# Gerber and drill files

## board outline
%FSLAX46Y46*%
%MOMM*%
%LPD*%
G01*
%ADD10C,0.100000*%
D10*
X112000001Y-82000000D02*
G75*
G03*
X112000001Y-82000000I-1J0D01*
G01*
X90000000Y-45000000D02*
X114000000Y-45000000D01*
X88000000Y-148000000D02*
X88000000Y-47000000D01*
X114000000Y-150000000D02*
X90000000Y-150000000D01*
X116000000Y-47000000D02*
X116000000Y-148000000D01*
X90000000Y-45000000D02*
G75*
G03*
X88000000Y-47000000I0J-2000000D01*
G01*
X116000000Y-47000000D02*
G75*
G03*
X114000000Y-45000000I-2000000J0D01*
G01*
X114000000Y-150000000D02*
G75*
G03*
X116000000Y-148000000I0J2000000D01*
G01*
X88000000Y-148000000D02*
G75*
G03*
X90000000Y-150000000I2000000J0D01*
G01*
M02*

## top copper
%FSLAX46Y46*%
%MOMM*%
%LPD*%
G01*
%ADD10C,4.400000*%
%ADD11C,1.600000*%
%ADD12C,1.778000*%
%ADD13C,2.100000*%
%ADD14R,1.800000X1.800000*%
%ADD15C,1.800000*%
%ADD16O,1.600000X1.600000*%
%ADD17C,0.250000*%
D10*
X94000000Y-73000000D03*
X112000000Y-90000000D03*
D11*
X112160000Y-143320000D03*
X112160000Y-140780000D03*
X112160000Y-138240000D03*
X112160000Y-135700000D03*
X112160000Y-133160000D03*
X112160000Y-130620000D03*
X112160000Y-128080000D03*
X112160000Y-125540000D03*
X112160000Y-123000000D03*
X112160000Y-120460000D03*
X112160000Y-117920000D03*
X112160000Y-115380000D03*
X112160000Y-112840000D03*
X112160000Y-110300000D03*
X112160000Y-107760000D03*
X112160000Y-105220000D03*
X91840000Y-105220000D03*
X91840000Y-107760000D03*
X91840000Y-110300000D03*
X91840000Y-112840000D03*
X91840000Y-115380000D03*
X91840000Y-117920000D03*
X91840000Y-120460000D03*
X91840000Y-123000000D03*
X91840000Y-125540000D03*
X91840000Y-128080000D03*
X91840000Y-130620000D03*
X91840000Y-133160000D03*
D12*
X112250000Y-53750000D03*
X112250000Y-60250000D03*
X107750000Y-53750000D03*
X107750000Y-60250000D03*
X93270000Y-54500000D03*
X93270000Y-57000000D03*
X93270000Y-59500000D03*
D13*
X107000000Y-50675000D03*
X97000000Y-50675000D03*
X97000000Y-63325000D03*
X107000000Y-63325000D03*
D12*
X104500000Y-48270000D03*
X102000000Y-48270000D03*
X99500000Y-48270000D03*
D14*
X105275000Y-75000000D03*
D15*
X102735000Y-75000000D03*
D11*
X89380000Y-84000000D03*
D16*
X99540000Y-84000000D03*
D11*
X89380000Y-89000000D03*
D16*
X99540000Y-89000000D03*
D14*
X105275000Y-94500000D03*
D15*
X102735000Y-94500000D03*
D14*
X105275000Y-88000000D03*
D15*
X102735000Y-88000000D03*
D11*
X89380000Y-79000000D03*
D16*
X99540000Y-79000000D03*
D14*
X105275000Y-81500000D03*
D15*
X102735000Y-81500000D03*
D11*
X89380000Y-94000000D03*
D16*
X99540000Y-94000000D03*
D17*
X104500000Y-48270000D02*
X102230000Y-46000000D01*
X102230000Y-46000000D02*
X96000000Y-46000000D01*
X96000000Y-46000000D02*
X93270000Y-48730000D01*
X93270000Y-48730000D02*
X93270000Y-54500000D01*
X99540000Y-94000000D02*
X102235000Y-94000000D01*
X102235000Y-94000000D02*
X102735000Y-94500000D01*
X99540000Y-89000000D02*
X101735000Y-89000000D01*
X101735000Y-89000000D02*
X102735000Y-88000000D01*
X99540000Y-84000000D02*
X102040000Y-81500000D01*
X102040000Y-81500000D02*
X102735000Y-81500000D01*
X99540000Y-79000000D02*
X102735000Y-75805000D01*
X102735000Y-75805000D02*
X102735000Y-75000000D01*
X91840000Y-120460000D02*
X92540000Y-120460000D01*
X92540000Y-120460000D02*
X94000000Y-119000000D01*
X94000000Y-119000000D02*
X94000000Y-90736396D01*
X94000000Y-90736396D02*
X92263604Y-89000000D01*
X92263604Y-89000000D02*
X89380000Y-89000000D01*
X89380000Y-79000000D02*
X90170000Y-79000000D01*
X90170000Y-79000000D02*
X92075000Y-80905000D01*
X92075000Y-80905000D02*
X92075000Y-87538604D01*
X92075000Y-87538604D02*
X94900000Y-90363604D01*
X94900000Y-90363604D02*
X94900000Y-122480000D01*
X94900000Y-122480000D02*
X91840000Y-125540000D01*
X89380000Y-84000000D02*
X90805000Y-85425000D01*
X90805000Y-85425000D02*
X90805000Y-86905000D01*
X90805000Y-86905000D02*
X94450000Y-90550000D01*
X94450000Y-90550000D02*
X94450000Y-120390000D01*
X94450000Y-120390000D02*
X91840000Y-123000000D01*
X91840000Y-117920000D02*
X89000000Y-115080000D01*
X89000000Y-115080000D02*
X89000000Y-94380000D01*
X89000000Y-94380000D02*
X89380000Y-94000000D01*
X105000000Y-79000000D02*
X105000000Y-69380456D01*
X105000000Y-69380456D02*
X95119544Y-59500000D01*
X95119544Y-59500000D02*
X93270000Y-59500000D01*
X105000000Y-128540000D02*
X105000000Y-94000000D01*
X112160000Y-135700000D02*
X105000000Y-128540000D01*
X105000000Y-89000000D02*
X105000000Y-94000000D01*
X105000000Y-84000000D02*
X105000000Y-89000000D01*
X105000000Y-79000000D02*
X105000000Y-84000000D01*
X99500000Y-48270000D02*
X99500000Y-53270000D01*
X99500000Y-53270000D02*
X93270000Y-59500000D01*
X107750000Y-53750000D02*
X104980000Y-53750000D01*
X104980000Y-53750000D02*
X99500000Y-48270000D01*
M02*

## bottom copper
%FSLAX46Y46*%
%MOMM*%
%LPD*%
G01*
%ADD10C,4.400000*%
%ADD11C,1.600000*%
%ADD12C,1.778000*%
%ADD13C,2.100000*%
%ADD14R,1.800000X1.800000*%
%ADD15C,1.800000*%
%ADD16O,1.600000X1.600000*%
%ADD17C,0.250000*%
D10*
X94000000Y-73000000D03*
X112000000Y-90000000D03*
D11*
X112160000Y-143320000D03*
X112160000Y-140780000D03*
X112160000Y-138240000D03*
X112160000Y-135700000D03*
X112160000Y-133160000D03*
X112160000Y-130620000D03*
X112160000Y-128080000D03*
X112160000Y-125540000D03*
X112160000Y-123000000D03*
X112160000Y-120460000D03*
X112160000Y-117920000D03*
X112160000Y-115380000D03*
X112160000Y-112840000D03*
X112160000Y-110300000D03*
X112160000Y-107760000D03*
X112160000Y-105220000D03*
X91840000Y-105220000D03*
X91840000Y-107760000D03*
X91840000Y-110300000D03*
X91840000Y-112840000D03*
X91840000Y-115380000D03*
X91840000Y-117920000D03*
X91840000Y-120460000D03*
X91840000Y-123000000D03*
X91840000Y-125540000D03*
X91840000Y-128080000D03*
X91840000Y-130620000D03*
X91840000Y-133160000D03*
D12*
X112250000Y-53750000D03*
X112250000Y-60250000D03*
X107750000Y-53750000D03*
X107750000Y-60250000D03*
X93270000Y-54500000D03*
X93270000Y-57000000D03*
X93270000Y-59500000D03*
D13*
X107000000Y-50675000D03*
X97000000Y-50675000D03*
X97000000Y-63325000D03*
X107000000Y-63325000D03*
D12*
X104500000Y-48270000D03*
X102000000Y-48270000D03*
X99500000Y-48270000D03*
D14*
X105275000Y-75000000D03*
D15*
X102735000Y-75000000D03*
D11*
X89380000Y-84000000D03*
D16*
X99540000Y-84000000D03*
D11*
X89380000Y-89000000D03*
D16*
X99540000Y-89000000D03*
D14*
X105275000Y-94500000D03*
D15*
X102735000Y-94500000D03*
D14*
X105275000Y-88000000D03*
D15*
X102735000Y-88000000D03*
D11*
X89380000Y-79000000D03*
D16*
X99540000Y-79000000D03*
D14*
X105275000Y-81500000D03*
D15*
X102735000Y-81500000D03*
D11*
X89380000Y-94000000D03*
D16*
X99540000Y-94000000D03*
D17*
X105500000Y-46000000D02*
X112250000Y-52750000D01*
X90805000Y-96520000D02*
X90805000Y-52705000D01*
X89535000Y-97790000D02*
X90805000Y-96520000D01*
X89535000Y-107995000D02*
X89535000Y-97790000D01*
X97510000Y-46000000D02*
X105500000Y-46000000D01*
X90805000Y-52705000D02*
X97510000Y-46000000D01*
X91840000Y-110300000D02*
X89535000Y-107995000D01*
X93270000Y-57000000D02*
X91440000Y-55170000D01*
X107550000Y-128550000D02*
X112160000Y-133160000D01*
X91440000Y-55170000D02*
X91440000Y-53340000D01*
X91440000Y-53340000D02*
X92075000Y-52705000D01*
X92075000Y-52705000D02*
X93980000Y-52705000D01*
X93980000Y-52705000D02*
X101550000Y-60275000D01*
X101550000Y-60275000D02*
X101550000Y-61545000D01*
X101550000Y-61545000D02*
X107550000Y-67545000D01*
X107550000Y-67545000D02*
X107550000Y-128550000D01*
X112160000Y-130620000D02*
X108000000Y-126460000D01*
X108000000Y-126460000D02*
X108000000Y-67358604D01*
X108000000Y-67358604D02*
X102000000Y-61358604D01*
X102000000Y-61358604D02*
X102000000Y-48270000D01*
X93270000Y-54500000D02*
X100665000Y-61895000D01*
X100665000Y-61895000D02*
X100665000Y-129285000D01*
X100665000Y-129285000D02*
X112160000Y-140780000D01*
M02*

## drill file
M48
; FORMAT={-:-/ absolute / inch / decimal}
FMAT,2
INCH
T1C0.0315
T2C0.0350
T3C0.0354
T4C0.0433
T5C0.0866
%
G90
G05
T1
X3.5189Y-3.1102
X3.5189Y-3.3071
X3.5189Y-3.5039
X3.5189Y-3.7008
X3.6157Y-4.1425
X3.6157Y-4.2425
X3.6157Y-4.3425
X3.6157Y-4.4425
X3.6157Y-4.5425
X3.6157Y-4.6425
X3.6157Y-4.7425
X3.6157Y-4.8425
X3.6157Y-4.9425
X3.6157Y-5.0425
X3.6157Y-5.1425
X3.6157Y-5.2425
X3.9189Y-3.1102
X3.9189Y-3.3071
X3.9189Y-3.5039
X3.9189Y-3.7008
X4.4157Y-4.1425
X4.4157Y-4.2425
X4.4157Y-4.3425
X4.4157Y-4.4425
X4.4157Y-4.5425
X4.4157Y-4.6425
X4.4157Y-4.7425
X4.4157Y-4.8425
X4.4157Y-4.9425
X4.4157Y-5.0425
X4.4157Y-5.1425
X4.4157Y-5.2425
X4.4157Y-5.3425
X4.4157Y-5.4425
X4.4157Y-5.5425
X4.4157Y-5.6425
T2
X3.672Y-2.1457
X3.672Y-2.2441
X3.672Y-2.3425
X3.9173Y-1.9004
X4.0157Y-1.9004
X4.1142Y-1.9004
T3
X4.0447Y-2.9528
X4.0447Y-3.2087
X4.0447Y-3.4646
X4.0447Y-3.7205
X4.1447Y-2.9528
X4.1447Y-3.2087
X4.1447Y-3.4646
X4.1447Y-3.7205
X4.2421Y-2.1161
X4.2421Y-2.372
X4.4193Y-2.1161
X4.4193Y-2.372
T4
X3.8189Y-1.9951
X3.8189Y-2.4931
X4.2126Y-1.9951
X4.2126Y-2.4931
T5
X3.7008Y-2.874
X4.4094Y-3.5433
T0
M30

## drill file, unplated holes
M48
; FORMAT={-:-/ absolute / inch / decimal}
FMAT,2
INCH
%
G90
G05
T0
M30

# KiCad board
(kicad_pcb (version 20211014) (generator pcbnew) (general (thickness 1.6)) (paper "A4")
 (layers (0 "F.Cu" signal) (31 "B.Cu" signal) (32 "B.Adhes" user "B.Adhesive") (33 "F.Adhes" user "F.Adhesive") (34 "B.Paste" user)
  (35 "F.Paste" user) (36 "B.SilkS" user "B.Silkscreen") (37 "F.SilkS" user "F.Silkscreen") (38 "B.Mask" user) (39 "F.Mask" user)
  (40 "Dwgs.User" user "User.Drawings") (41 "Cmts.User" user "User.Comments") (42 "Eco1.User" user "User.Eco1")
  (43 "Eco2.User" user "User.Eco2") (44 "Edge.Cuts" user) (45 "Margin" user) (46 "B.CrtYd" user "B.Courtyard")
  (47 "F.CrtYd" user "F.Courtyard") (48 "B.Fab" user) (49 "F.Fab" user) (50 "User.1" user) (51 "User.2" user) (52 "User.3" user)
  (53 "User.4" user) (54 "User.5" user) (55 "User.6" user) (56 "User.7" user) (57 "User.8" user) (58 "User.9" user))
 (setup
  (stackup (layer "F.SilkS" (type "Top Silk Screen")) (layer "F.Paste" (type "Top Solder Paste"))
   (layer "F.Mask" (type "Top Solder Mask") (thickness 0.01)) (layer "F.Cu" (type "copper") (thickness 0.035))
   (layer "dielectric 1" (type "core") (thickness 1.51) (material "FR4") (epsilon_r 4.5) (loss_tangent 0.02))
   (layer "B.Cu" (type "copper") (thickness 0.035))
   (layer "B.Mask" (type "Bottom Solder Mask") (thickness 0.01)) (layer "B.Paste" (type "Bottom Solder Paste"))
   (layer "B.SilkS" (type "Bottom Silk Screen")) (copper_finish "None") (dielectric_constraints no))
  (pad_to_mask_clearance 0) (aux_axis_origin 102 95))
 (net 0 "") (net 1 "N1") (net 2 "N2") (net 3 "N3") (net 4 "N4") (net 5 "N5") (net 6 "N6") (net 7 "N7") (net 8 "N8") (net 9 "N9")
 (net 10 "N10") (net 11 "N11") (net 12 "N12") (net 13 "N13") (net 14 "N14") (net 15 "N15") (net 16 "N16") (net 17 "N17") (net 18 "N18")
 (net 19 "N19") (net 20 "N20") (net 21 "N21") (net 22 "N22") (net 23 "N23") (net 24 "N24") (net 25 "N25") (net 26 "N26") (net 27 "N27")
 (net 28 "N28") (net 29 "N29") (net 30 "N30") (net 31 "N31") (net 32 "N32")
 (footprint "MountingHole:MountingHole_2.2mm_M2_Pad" (layer "F.Cu") (at 94 73)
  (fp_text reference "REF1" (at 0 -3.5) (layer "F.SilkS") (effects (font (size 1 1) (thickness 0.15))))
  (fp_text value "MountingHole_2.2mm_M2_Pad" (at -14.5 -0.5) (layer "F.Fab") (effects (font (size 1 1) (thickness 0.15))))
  (pad "1" thru_hole circle (at 0 0) (size 4.4 4.4) (drill 2.2) (layers *.Cu *.Mask)))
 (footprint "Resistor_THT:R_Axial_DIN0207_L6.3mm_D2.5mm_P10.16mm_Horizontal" (layer "F.Cu") (at 89.38 84)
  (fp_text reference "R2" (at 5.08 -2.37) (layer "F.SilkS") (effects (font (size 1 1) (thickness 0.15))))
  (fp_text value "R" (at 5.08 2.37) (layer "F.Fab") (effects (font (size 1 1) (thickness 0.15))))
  (pad "1" thru_hole circle (at 0 0) (size 1.6 1.6) (drill 0.8) (layers *.Cu *.Mask) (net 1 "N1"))
  (pad "2" thru_hole oval (at 10.16 0) (size 1.6 1.6) (drill 0.8) (layers *.Cu *.Mask) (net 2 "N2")))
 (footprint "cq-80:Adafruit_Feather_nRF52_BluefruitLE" (layer "F.Cu") (at 102 123 180)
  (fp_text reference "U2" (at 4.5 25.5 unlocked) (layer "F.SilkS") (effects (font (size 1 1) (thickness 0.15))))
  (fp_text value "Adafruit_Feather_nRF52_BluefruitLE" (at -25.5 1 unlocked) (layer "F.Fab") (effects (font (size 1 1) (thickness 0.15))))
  (pad "1" thru_hole circle (at -10.16 -20.32) (size 1.6 1.6) (drill 0.8) (layers *.Cu *.Mask) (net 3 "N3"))
  (pad "2" thru_hole circle (at -10.16 -17.78) (size 1.6 1.6) (drill 0.8) (layers *.Cu *.Mask) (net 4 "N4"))
  (pad "3" thru_hole circle (at -10.16 -15.24) (size 1.6 1.6) (drill 0.8) (layers *.Cu *.Mask) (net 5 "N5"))
  (pad "4" thru_hole circle (at -10.16 -12.7) (size 1.6 1.6) (drill 0.8) (layers *.Cu *.Mask) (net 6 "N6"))
  (pad "5" thru_hole circle (at -10.16 -10.16) (size 1.6 1.6) (drill 0.8) (layers *.Cu *.Mask) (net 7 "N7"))
  (pad "6" thru_hole circle (at -10.16 -7.62) (size 1.6 1.6) (drill 0.8) (layers *.Cu *.Mask) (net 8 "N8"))
  (pad "7" thru_hole circle (at -10.16 -5.08) (size 1.6 1.6) (drill 0.8) (layers *.Cu *.Mask) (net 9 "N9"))
  (pad "8" thru_hole circle (at -10.16 -2.54) (size 1.6 1.6) (drill 0.8) (layers *.Cu *.Mask) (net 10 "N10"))
  (pad "9" thru_hole circle (at -10.16 0) (size 1.6 1.6) (drill 0.8) (layers *.Cu *.Mask) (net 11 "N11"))
  (pad "10" thru_hole circle (at -10.16 2.54) (size 1.6 1.6) (drill 0.8) (layers *.Cu *.Mask) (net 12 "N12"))
  (pad "11" thru_hole circle (at -10.16 5.08) (size 1.6 1.6) (drill 0.8) (layers *.Cu *.Mask) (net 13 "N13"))
  (pad "12" thru_hole circle (at -10.16 7.62) (size 1.6 1.6) (drill 0.8) (layers *.Cu *.Mask) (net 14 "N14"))
  (pad "13" thru_hole circle (at -10.16 10.16) (size 1.6 1.6) (drill 0.8) (layers *.Cu *.Mask) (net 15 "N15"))
  (pad "14" thru_hole circle (at -10.16 12.7) (size 1.6 1.6) (drill 0.8) (layers *.Cu *.Mask) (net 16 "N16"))
  (pad "15" thru_hole circle (at -10.16 15.24) (size 1.6 1.6) (drill 0.8) (layers *.Cu *.Mask) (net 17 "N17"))
  (pad "16" thru_hole circle (at -10.16 17.78) (size 1.6 1.6) (drill 0.8) (layers *.Cu *.Mask) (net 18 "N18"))
  (pad "17" thru_hole circle (at 10.16 17.78) (size 1.6 1.6) (drill 0.8) (layers *.Cu *.Mask) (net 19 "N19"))
  (pad "18" thru_hole circle (at 10.16 15.24) (size 1.6 1.6) (drill 0.8) (layers *.Cu *.Mask) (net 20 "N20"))
  (pad "19" thru_hole circle (at 10.16 12.7) (size 1.6 1.6) (drill 0.8) (layers *.Cu *.Mask) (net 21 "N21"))
  (pad "20" thru_hole circle (at 10.16 10.16) (size 1.6 1.6) (drill 0.8) (layers *.Cu *.Mask) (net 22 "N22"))
  (pad "21" thru_hole circle (at 10.16 7.62) (size 1.6 1.6) (drill 0.8) (layers *.Cu *.Mask) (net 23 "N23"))
  (pad "22" thru_hole circle (at 10.16 5.08) (size 1.6 1.6) (drill 0.8) (layers *.Cu *.Mask) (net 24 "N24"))
  (pad "23" thru_hole circle (at 10.16 2.54) (size 1.6 1.6) (drill 0.8) (layers *.Cu *.Mask) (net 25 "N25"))
  (pad "24" thru_hole circle (at 10.16 0) (size 1.6 1.6) (drill 0.8) (layers *.Cu *.Mask) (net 1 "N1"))
  (pad "25" thru_hole circle (at 10.16 -2.54) (size 1.6 1.6) (drill 0.8) (layers *.Cu *.Mask) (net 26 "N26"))
  (pad "26" thru_hole circle (at 10.16 -5.08) (size 1.6 1.6) (drill 0.8) (layers *.Cu *.Mask) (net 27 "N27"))
  (pad "27" thru_hole circle (at 10.16 -7.62) (size 1.6 1.6) (drill 0.8) (layers *.Cu *.Mask) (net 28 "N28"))
  (pad "28" thru_hole circle (at 10.16 -10.16) (size 1.6 1.6) (drill 0.8) (layers *.Cu *.Mask) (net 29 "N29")))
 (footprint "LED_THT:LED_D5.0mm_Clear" (layer "F.Cu") (at 105.275 75 180)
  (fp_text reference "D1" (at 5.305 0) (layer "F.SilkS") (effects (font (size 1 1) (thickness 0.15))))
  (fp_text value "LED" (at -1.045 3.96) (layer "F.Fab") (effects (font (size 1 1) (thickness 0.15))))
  (pad "1" thru_hole rect (at 0 0 180) (size 1.8 1.8) (drill 0.9) (layers *.Cu *.Mask) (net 6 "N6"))
  (pad "2" thru_hole circle (at 2.54 0 180) (size 1.8 1.8) (drill 0.9) (layers *.Cu *.Mask) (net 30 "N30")))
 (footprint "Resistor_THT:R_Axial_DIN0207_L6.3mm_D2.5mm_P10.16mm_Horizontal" (layer "F.Cu") (at 89.38 89)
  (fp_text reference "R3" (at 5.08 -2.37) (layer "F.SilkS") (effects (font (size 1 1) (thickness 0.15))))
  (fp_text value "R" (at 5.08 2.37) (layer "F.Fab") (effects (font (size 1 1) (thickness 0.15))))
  (pad "1" thru_hole circle (at 0 0) (size 1.6 1.6) (drill 0.8) (layers *.Cu *.Mask) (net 25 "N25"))
  (pad "2" thru_hole oval (at 10.16 0) (size 1.6 1.6) (drill 0.8) (layers *.Cu *.Mask) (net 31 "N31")))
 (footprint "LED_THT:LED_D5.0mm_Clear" (layer "F.Cu") (at 105.275 94.5 180)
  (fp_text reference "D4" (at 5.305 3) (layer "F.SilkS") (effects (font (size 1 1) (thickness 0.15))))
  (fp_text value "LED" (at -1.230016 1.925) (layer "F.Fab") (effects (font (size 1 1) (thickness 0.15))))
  (pad "1" thru_hole rect (at 0 0 180) (size 1.8 1.8) (drill 0.9) (layers *.Cu *.Mask) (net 6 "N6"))
  (pad "2" thru_hole circle (at 2.54 0 180) (size 1.8 1.8) (drill 0.9) (layers *.Cu *.Mask) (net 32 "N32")))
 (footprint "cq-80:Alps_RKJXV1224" (layer "F.Cu") (at 102 57 -90)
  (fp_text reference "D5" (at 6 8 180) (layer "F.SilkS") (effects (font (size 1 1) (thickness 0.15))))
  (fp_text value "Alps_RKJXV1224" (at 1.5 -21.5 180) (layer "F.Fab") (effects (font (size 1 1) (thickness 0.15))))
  (pad "B1A" thru_hole circle (at -3.25 -10.25 270) (size 1.778 1.778) (drill 0.9) (layers *.Cu *.Mask) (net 21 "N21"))
  (pad "B1B" thru_hole circle (at 3.25 -10.25 270) (size 1.778 1.778) (drill 0.9) (layers *.Cu *.Mask))
  (pad "B2A" thru_hole circle (at -3.25 -5.75 270) (size 1.778 1.778) (drill 0.9) (layers *.Cu *.Mask) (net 6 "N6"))
  (pad "B2B" thru_hole circle (at 3.25 -5.75 270) (size 1.778 1.778) (drill 0.9) (layers *.Cu *.Mask))
  (pad "H1" thru_hole circle (at -2.5 8.73 270) (size 1.778 1.778) (drill 0.889) (layers *.Cu *.Mask) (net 4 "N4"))
  (pad "H2" thru_hole circle (at 0 8.73 270) (size 1.778 1.778) (drill 0.889) (layers *.Cu *.Mask) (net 7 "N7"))
  (pad "H3" thru_hole circle (at 2.5 8.73 270) (size 1.778 1.778) (drill 0.889) (layers *.Cu *.Mask) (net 6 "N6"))
  (pad "S1" thru_hole circle (at -6.325 -5 270) (size 2.1 2.1) (drill 1.1) (layers *.Cu *.Mask))
  (pad "S2" thru_hole circle (at -6.325 5 270) (size 2.1 2.1) (drill 1.1) (layers *.Cu *.Mask))
  (pad "S3" thru_hole circle (at 6.325 5 270) (size 2.1 2.1) (drill 1.1) (layers *.Cu *.Mask))
  (pad "S4" thru_hole circle (at 6.325 -5 270) (size 2.1 2.1) (drill 1.1) (layers *.Cu *.Mask))
  (pad "V1" thru_hole circle (at -8.73 -2.5 270) (size 1.778 1.778) (drill 0.889) (layers *.Cu *.Mask) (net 4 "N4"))
  (pad "V2" thru_hole circle (at -8.73 0 270) (size 1.778 1.778) (drill 0.889) (layers *.Cu *.Mask) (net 8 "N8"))
  (pad "V3" thru_hole circle (at -8.73 2.5 270) (size 1.778 1.778) (drill 0.889) (layers *.Cu *.Mask) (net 6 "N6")))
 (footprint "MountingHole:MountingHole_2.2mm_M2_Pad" (layer "F.Cu") (at 112 90)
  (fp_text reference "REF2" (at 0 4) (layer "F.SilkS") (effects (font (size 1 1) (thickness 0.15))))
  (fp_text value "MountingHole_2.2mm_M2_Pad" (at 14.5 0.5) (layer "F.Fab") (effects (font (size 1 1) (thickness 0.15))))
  (pad "1" thru_hole circle (at 0 0) (size 4.4 4.4) (drill 2.2) (layers *.Cu *.Mask)))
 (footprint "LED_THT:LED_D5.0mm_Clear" (layer "F.Cu") (at 105.275 88 180)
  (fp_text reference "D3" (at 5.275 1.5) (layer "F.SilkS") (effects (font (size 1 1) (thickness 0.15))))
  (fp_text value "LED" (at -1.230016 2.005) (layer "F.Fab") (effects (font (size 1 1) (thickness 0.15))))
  (pad "1" thru_hole rect (at 0 0 180) (size 1.8 1.8) (drill 0.9) (layers *.Cu *.Mask) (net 6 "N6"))
  (pad "2" thru_hole circle (at 2.54 0 180) (size 1.8 1.8) (drill 0.9) (layers *.Cu *.Mask) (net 31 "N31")))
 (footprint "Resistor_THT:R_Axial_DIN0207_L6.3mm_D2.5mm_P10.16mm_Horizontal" (layer "F.Cu") (at 89.38 79)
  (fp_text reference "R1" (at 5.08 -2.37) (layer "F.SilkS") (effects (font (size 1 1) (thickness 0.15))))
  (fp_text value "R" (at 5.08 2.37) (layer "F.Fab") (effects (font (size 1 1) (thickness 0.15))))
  (pad "1" thru_hole circle (at 0 0) (size 1.6 1.6) (drill 0.8) (layers *.Cu *.Mask) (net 26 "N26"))
  (pad "2" thru_hole oval (at 10.16 0) (size 1.6 1.6) (drill 0.8) (layers *.Cu *.Mask) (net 30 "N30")))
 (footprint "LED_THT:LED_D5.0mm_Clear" (layer "F.Cu") (at 105.275 81.5 180)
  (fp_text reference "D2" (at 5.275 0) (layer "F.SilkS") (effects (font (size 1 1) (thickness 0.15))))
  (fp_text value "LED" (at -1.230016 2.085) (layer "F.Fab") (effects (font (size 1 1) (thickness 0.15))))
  (pad "1" thru_hole rect (at 0 0 180) (size 1.8 1.8) (drill 0.9) (layers *.Cu *.Mask) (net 6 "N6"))
  (pad "2" thru_hole circle (at 2.54 0 180) (size 1.8 1.8) (drill 0.9) (layers *.Cu *.Mask) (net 2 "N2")))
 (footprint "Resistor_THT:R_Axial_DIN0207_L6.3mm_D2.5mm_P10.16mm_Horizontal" (layer "F.Cu") (at 89.38 94)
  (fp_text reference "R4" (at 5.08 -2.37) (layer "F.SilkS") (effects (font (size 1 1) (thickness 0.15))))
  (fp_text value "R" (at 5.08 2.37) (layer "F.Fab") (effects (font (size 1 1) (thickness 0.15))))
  (pad "1" thru_hole circle (at 0 0) (size 1.6 1.6) (drill 0.8) (layers *.Cu *.Mask) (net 24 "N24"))
  (pad "2" thru_hole oval (at 10.16 0) (size 1.6 1.6) (drill 0.8) (layers *.Cu *.Mask) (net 32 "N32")))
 (gr_arc (start 116 148) (mid 115.414214 149.414214) (end 114 150) (layer "Edge.Cuts") (width 0.1))
 (gr_arc (start 88 47) (mid 88.585786 45.585786) (end 90 45) (layer "Edge.Cuts") (width 0.1))
 (gr_line (start 88 148) (end 88 47) (layer "Edge.Cuts") (width 0.1))
 (gr_circle (center 112 82) (end 112 82) (layer "Edge.Cuts") (width 0.1) (fill none))
 (gr_line (start 116 47) (end 116 148) (layer "Edge.Cuts") (width 0.1))
 (gr_line (start 90 45) (end 114 45) (layer "Edge.Cuts") (width 0.1))
 (gr_arc (start 90 150) (mid 88.585786 149.414214) (end 88 148) (layer "Edge.Cuts") (width 0.1))
 (gr_arc (start 114 45) (mid 115.414214 45.585786) (end 116 47) (layer "Edge.Cuts") (width 0.1))
 (gr_line (start 114 150) (end 90 150) (layer "Edge.Cuts") (width 0.1))
 (segment (start 105 128.54) (end 105 94) (width 0.25) (layer "F.Cu") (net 6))
 (segment (start 105 79) (end 105 69.380456) (width 0.25) (layer "F.Cu") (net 6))
 (segment (start 95.119544 59.5) (end 93.27 59.5) (width 0.25) (layer "F.Cu") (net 6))
 (segment (start 107.75 53.75) (end 104.98 53.75) (width 0.25) (layer "F.Cu") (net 6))
 (segment (start 105 89) (end 105 94) (width 0.25) (layer "F.Cu") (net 6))
 (segment (start 99.5 48.27) (end 99.5 53.27) (width 0.25) (layer "F.Cu") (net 6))
 (segment (start 105 79) (end 105 84) (width 0.25) (layer "F.Cu") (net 6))
 (segment (start 112.16 135.7) (end 105 128.54) (width 0.25) (layer "F.Cu") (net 6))
 (segment (start 104.98 53.75) (end 99.5 48.27) (width 0.25) (layer "F.Cu") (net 6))
 (segment (start 99.5 53.27) (end 93.27 59.5) (width 0.25) (layer "F.Cu") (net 6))
 (segment (start 105 84) (end 105 89) (width 0.25) (layer "F.Cu") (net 6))
 (segment (start 105 69.380456) (end 95.119544 59.5) (width 0.25) (layer "F.Cu") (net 6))
 (segment (start 105.5 46) (end 112.25 52.75) (width 0.25) (layer "B.Cu") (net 21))
 (segment (start 97.51 46) (end 105.5 46) (width 0.25) (layer "B.Cu") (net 21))
 (segment (start 91.84 110.3) (end 89.535 107.995) (width 0.25) (layer "B.Cu") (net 21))
 (segment (start 89.535 97.79) (end 90.805 96.52) (width 0.25) (layer "B.Cu") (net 21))
 (segment (start 89.535 107.995) (end 89.535 97.79) (width 0.25) (layer "B.Cu") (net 21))
 (segment (start 90.805 96.52) (end 90.805 52.705) (width 0.25) (layer "B.Cu") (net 21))
 (segment (start 90.805 52.705) (end 97.51 46) (width 0.25) (layer "B.Cu") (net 21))
 (segment (start 102.23 46) (end 96 46) (width 0.25) (layer "F.Cu") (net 4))
 (segment (start 93.27 48.73) (end 93.27 54.5) (width 0.25) (layer "F.Cu") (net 4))
 (segment (start 104.5 48.27) (end 102.23 46) (width 0.25) (layer "F.Cu") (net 4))
 (segment (start 96 46) (end 93.27 48.73) (width 0.25) (layer "F.Cu") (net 4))
 (segment (start 93.27 54.5) (end 100.665 61.895) (width 0.25) (layer "B.Cu") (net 4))
 (segment (start 100.665 129.285) (end 112.16 140.78) (width 0.25) (layer "B.Cu") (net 4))
 (segment (start 100.665 61.895) (end 100.665 129.285) (width 0.25) (layer "B.Cu") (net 4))
 (segment (start 93.98 52.705) (end 101.55 60.275) (width 0.25) (layer "B.Cu") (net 7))
 (segment (start 93.27 57) (end 91.44 55.17) (width 0.25) (layer "B.Cu") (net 7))
 (segment (start 91.44 53.34) (end 92.075 52.705) (width 0.25) (layer "B.Cu") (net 7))
 (segment (start 101.55 61.545) (end 107.55 67.545) (width 0.25) (layer "B.Cu") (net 7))
 (segment (start 101.55 60.275) (end 101.55 61.545) (width 0.25) (layer "B.Cu") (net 7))
 (segment (start 107.55 128.55) (end 112.16 133.16) (width 0.25) (layer "B.Cu") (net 7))
 (segment (start 92.075 52.705) (end 93.98 52.705) (width 0.25) (layer "B.Cu") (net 7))
 (segment (start 91.44 55.17) (end 91.44 53.34) (width 0.25) (layer "B.Cu") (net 7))
 (segment (start 107.55 67.545) (end 107.55 128.55) (width 0.25) (layer "B.Cu") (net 7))
 (segment (start 102 61.358604) (end 102 48.27) (width 0.25) (layer "B.Cu") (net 8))
 (segment (start 108 126.46) (end 108 67.358604) (width 0.25) (layer "B.Cu") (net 8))
 (segment (start 108 67.358604) (end 102 61.358604) (width 0.25) (layer "B.Cu") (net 8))
 (segment (start 112.16 130.62) (end 108 126.46) (width 0.25) (layer "B.Cu") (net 8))
 (segment (start 102.735 75.805) (end 102.735 75) (width 0.25) (layer "F.Cu") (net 30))
 (segment (start 99.54 79) (end 102.735 75.805) (width 0.25) (layer "F.Cu") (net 30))
 (segment (start 99.54 84) (end 102.04 81.5) (width 0.25) (layer "F.Cu") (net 2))
 (segment (start 102.04 81.5) (end 102.735 81.5) (width 0.25) (layer "F.Cu") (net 2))
 (segment (start 99.54 89) (end 101.735 89) (width 0.25) (layer "F.Cu") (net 31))
 (segment (start 101.735 89) (end 102.735 88) (width 0.25) (layer "F.Cu") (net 31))
 (segment (start 99.54 94) (end 102.235 94) (width 0.25) (layer "F.Cu") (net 32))
 (segment (start 102.235 94) (end 102.735 94.5) (width 0.25) (layer "F.Cu") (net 32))
 (segment (start 89.38 79) (end 90.17 79) (width 0.25) (layer "F.Cu") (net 26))
 (segment (start 90.17 79) (end 92.075 80.905) (width 0.25) (layer "F.Cu") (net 26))
 (segment (start 92.075 87.538604) (end 94.9 90.363604) (width 0.25) (layer "F.Cu") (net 26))
 (segment (start 92.075 80.905) (end 92.075 87.538604) (width 0.25) (layer "F.Cu") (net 26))
 (segment (start 94.9 90.363604) (end 94.9 122.48) (width 0.25) (layer "F.Cu") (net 26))
 (segment (start 94.9 122.48) (end 91.84 125.54) (width 0.25) (layer "F.Cu") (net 26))
 (segment (start 90.805 86.905) (end 94.45 90.55) (width 0.25) (layer "F.Cu") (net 1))
 (segment (start 90.805 85.425) (end 90.805 86.905) (width 0.25) (layer "F.Cu") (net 1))
 (segment (start 89.38 84) (end 90.805 85.425) (width 0.25) (layer "F.Cu") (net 1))
 (segment (start 94.45 90.55) (end 94.45 120.39) (width 0.25) (layer "F.Cu") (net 1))
 (segment (start 94.45 120.39) (end 91.84 123) (width 0.25) (layer "F.Cu") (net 1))
 (segment (start 92.263604 89) (end 89.38 89) (width 0.25) (layer "F.Cu") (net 25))
 (segment (start 92.54 120.46) (end 94 119) (width 0.25) (layer "F.Cu") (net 25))
 (segment (start 94 90.736396) (end 92.263604 89) (width 0.25) (layer "F.Cu") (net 25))
 (segment (start 94 119) (end 94 90.736396) (width 0.25) (layer "F.Cu") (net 25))
 (segment (start 91.84 120.46) (end 92.54 120.46) (width 0.25) (layer "F.Cu") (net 25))
 (segment (start 89 115.08) (end 89 94.38) (width 0.25) (layer "F.Cu") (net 24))
 (segment (start 91.84 117.92) (end 89 115.08) (width 0.25) (layer "F.Cu") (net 24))
 (segment (start 89 94.38) (end 89.38 94) (width 0.25) (layer "F.Cu") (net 24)))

